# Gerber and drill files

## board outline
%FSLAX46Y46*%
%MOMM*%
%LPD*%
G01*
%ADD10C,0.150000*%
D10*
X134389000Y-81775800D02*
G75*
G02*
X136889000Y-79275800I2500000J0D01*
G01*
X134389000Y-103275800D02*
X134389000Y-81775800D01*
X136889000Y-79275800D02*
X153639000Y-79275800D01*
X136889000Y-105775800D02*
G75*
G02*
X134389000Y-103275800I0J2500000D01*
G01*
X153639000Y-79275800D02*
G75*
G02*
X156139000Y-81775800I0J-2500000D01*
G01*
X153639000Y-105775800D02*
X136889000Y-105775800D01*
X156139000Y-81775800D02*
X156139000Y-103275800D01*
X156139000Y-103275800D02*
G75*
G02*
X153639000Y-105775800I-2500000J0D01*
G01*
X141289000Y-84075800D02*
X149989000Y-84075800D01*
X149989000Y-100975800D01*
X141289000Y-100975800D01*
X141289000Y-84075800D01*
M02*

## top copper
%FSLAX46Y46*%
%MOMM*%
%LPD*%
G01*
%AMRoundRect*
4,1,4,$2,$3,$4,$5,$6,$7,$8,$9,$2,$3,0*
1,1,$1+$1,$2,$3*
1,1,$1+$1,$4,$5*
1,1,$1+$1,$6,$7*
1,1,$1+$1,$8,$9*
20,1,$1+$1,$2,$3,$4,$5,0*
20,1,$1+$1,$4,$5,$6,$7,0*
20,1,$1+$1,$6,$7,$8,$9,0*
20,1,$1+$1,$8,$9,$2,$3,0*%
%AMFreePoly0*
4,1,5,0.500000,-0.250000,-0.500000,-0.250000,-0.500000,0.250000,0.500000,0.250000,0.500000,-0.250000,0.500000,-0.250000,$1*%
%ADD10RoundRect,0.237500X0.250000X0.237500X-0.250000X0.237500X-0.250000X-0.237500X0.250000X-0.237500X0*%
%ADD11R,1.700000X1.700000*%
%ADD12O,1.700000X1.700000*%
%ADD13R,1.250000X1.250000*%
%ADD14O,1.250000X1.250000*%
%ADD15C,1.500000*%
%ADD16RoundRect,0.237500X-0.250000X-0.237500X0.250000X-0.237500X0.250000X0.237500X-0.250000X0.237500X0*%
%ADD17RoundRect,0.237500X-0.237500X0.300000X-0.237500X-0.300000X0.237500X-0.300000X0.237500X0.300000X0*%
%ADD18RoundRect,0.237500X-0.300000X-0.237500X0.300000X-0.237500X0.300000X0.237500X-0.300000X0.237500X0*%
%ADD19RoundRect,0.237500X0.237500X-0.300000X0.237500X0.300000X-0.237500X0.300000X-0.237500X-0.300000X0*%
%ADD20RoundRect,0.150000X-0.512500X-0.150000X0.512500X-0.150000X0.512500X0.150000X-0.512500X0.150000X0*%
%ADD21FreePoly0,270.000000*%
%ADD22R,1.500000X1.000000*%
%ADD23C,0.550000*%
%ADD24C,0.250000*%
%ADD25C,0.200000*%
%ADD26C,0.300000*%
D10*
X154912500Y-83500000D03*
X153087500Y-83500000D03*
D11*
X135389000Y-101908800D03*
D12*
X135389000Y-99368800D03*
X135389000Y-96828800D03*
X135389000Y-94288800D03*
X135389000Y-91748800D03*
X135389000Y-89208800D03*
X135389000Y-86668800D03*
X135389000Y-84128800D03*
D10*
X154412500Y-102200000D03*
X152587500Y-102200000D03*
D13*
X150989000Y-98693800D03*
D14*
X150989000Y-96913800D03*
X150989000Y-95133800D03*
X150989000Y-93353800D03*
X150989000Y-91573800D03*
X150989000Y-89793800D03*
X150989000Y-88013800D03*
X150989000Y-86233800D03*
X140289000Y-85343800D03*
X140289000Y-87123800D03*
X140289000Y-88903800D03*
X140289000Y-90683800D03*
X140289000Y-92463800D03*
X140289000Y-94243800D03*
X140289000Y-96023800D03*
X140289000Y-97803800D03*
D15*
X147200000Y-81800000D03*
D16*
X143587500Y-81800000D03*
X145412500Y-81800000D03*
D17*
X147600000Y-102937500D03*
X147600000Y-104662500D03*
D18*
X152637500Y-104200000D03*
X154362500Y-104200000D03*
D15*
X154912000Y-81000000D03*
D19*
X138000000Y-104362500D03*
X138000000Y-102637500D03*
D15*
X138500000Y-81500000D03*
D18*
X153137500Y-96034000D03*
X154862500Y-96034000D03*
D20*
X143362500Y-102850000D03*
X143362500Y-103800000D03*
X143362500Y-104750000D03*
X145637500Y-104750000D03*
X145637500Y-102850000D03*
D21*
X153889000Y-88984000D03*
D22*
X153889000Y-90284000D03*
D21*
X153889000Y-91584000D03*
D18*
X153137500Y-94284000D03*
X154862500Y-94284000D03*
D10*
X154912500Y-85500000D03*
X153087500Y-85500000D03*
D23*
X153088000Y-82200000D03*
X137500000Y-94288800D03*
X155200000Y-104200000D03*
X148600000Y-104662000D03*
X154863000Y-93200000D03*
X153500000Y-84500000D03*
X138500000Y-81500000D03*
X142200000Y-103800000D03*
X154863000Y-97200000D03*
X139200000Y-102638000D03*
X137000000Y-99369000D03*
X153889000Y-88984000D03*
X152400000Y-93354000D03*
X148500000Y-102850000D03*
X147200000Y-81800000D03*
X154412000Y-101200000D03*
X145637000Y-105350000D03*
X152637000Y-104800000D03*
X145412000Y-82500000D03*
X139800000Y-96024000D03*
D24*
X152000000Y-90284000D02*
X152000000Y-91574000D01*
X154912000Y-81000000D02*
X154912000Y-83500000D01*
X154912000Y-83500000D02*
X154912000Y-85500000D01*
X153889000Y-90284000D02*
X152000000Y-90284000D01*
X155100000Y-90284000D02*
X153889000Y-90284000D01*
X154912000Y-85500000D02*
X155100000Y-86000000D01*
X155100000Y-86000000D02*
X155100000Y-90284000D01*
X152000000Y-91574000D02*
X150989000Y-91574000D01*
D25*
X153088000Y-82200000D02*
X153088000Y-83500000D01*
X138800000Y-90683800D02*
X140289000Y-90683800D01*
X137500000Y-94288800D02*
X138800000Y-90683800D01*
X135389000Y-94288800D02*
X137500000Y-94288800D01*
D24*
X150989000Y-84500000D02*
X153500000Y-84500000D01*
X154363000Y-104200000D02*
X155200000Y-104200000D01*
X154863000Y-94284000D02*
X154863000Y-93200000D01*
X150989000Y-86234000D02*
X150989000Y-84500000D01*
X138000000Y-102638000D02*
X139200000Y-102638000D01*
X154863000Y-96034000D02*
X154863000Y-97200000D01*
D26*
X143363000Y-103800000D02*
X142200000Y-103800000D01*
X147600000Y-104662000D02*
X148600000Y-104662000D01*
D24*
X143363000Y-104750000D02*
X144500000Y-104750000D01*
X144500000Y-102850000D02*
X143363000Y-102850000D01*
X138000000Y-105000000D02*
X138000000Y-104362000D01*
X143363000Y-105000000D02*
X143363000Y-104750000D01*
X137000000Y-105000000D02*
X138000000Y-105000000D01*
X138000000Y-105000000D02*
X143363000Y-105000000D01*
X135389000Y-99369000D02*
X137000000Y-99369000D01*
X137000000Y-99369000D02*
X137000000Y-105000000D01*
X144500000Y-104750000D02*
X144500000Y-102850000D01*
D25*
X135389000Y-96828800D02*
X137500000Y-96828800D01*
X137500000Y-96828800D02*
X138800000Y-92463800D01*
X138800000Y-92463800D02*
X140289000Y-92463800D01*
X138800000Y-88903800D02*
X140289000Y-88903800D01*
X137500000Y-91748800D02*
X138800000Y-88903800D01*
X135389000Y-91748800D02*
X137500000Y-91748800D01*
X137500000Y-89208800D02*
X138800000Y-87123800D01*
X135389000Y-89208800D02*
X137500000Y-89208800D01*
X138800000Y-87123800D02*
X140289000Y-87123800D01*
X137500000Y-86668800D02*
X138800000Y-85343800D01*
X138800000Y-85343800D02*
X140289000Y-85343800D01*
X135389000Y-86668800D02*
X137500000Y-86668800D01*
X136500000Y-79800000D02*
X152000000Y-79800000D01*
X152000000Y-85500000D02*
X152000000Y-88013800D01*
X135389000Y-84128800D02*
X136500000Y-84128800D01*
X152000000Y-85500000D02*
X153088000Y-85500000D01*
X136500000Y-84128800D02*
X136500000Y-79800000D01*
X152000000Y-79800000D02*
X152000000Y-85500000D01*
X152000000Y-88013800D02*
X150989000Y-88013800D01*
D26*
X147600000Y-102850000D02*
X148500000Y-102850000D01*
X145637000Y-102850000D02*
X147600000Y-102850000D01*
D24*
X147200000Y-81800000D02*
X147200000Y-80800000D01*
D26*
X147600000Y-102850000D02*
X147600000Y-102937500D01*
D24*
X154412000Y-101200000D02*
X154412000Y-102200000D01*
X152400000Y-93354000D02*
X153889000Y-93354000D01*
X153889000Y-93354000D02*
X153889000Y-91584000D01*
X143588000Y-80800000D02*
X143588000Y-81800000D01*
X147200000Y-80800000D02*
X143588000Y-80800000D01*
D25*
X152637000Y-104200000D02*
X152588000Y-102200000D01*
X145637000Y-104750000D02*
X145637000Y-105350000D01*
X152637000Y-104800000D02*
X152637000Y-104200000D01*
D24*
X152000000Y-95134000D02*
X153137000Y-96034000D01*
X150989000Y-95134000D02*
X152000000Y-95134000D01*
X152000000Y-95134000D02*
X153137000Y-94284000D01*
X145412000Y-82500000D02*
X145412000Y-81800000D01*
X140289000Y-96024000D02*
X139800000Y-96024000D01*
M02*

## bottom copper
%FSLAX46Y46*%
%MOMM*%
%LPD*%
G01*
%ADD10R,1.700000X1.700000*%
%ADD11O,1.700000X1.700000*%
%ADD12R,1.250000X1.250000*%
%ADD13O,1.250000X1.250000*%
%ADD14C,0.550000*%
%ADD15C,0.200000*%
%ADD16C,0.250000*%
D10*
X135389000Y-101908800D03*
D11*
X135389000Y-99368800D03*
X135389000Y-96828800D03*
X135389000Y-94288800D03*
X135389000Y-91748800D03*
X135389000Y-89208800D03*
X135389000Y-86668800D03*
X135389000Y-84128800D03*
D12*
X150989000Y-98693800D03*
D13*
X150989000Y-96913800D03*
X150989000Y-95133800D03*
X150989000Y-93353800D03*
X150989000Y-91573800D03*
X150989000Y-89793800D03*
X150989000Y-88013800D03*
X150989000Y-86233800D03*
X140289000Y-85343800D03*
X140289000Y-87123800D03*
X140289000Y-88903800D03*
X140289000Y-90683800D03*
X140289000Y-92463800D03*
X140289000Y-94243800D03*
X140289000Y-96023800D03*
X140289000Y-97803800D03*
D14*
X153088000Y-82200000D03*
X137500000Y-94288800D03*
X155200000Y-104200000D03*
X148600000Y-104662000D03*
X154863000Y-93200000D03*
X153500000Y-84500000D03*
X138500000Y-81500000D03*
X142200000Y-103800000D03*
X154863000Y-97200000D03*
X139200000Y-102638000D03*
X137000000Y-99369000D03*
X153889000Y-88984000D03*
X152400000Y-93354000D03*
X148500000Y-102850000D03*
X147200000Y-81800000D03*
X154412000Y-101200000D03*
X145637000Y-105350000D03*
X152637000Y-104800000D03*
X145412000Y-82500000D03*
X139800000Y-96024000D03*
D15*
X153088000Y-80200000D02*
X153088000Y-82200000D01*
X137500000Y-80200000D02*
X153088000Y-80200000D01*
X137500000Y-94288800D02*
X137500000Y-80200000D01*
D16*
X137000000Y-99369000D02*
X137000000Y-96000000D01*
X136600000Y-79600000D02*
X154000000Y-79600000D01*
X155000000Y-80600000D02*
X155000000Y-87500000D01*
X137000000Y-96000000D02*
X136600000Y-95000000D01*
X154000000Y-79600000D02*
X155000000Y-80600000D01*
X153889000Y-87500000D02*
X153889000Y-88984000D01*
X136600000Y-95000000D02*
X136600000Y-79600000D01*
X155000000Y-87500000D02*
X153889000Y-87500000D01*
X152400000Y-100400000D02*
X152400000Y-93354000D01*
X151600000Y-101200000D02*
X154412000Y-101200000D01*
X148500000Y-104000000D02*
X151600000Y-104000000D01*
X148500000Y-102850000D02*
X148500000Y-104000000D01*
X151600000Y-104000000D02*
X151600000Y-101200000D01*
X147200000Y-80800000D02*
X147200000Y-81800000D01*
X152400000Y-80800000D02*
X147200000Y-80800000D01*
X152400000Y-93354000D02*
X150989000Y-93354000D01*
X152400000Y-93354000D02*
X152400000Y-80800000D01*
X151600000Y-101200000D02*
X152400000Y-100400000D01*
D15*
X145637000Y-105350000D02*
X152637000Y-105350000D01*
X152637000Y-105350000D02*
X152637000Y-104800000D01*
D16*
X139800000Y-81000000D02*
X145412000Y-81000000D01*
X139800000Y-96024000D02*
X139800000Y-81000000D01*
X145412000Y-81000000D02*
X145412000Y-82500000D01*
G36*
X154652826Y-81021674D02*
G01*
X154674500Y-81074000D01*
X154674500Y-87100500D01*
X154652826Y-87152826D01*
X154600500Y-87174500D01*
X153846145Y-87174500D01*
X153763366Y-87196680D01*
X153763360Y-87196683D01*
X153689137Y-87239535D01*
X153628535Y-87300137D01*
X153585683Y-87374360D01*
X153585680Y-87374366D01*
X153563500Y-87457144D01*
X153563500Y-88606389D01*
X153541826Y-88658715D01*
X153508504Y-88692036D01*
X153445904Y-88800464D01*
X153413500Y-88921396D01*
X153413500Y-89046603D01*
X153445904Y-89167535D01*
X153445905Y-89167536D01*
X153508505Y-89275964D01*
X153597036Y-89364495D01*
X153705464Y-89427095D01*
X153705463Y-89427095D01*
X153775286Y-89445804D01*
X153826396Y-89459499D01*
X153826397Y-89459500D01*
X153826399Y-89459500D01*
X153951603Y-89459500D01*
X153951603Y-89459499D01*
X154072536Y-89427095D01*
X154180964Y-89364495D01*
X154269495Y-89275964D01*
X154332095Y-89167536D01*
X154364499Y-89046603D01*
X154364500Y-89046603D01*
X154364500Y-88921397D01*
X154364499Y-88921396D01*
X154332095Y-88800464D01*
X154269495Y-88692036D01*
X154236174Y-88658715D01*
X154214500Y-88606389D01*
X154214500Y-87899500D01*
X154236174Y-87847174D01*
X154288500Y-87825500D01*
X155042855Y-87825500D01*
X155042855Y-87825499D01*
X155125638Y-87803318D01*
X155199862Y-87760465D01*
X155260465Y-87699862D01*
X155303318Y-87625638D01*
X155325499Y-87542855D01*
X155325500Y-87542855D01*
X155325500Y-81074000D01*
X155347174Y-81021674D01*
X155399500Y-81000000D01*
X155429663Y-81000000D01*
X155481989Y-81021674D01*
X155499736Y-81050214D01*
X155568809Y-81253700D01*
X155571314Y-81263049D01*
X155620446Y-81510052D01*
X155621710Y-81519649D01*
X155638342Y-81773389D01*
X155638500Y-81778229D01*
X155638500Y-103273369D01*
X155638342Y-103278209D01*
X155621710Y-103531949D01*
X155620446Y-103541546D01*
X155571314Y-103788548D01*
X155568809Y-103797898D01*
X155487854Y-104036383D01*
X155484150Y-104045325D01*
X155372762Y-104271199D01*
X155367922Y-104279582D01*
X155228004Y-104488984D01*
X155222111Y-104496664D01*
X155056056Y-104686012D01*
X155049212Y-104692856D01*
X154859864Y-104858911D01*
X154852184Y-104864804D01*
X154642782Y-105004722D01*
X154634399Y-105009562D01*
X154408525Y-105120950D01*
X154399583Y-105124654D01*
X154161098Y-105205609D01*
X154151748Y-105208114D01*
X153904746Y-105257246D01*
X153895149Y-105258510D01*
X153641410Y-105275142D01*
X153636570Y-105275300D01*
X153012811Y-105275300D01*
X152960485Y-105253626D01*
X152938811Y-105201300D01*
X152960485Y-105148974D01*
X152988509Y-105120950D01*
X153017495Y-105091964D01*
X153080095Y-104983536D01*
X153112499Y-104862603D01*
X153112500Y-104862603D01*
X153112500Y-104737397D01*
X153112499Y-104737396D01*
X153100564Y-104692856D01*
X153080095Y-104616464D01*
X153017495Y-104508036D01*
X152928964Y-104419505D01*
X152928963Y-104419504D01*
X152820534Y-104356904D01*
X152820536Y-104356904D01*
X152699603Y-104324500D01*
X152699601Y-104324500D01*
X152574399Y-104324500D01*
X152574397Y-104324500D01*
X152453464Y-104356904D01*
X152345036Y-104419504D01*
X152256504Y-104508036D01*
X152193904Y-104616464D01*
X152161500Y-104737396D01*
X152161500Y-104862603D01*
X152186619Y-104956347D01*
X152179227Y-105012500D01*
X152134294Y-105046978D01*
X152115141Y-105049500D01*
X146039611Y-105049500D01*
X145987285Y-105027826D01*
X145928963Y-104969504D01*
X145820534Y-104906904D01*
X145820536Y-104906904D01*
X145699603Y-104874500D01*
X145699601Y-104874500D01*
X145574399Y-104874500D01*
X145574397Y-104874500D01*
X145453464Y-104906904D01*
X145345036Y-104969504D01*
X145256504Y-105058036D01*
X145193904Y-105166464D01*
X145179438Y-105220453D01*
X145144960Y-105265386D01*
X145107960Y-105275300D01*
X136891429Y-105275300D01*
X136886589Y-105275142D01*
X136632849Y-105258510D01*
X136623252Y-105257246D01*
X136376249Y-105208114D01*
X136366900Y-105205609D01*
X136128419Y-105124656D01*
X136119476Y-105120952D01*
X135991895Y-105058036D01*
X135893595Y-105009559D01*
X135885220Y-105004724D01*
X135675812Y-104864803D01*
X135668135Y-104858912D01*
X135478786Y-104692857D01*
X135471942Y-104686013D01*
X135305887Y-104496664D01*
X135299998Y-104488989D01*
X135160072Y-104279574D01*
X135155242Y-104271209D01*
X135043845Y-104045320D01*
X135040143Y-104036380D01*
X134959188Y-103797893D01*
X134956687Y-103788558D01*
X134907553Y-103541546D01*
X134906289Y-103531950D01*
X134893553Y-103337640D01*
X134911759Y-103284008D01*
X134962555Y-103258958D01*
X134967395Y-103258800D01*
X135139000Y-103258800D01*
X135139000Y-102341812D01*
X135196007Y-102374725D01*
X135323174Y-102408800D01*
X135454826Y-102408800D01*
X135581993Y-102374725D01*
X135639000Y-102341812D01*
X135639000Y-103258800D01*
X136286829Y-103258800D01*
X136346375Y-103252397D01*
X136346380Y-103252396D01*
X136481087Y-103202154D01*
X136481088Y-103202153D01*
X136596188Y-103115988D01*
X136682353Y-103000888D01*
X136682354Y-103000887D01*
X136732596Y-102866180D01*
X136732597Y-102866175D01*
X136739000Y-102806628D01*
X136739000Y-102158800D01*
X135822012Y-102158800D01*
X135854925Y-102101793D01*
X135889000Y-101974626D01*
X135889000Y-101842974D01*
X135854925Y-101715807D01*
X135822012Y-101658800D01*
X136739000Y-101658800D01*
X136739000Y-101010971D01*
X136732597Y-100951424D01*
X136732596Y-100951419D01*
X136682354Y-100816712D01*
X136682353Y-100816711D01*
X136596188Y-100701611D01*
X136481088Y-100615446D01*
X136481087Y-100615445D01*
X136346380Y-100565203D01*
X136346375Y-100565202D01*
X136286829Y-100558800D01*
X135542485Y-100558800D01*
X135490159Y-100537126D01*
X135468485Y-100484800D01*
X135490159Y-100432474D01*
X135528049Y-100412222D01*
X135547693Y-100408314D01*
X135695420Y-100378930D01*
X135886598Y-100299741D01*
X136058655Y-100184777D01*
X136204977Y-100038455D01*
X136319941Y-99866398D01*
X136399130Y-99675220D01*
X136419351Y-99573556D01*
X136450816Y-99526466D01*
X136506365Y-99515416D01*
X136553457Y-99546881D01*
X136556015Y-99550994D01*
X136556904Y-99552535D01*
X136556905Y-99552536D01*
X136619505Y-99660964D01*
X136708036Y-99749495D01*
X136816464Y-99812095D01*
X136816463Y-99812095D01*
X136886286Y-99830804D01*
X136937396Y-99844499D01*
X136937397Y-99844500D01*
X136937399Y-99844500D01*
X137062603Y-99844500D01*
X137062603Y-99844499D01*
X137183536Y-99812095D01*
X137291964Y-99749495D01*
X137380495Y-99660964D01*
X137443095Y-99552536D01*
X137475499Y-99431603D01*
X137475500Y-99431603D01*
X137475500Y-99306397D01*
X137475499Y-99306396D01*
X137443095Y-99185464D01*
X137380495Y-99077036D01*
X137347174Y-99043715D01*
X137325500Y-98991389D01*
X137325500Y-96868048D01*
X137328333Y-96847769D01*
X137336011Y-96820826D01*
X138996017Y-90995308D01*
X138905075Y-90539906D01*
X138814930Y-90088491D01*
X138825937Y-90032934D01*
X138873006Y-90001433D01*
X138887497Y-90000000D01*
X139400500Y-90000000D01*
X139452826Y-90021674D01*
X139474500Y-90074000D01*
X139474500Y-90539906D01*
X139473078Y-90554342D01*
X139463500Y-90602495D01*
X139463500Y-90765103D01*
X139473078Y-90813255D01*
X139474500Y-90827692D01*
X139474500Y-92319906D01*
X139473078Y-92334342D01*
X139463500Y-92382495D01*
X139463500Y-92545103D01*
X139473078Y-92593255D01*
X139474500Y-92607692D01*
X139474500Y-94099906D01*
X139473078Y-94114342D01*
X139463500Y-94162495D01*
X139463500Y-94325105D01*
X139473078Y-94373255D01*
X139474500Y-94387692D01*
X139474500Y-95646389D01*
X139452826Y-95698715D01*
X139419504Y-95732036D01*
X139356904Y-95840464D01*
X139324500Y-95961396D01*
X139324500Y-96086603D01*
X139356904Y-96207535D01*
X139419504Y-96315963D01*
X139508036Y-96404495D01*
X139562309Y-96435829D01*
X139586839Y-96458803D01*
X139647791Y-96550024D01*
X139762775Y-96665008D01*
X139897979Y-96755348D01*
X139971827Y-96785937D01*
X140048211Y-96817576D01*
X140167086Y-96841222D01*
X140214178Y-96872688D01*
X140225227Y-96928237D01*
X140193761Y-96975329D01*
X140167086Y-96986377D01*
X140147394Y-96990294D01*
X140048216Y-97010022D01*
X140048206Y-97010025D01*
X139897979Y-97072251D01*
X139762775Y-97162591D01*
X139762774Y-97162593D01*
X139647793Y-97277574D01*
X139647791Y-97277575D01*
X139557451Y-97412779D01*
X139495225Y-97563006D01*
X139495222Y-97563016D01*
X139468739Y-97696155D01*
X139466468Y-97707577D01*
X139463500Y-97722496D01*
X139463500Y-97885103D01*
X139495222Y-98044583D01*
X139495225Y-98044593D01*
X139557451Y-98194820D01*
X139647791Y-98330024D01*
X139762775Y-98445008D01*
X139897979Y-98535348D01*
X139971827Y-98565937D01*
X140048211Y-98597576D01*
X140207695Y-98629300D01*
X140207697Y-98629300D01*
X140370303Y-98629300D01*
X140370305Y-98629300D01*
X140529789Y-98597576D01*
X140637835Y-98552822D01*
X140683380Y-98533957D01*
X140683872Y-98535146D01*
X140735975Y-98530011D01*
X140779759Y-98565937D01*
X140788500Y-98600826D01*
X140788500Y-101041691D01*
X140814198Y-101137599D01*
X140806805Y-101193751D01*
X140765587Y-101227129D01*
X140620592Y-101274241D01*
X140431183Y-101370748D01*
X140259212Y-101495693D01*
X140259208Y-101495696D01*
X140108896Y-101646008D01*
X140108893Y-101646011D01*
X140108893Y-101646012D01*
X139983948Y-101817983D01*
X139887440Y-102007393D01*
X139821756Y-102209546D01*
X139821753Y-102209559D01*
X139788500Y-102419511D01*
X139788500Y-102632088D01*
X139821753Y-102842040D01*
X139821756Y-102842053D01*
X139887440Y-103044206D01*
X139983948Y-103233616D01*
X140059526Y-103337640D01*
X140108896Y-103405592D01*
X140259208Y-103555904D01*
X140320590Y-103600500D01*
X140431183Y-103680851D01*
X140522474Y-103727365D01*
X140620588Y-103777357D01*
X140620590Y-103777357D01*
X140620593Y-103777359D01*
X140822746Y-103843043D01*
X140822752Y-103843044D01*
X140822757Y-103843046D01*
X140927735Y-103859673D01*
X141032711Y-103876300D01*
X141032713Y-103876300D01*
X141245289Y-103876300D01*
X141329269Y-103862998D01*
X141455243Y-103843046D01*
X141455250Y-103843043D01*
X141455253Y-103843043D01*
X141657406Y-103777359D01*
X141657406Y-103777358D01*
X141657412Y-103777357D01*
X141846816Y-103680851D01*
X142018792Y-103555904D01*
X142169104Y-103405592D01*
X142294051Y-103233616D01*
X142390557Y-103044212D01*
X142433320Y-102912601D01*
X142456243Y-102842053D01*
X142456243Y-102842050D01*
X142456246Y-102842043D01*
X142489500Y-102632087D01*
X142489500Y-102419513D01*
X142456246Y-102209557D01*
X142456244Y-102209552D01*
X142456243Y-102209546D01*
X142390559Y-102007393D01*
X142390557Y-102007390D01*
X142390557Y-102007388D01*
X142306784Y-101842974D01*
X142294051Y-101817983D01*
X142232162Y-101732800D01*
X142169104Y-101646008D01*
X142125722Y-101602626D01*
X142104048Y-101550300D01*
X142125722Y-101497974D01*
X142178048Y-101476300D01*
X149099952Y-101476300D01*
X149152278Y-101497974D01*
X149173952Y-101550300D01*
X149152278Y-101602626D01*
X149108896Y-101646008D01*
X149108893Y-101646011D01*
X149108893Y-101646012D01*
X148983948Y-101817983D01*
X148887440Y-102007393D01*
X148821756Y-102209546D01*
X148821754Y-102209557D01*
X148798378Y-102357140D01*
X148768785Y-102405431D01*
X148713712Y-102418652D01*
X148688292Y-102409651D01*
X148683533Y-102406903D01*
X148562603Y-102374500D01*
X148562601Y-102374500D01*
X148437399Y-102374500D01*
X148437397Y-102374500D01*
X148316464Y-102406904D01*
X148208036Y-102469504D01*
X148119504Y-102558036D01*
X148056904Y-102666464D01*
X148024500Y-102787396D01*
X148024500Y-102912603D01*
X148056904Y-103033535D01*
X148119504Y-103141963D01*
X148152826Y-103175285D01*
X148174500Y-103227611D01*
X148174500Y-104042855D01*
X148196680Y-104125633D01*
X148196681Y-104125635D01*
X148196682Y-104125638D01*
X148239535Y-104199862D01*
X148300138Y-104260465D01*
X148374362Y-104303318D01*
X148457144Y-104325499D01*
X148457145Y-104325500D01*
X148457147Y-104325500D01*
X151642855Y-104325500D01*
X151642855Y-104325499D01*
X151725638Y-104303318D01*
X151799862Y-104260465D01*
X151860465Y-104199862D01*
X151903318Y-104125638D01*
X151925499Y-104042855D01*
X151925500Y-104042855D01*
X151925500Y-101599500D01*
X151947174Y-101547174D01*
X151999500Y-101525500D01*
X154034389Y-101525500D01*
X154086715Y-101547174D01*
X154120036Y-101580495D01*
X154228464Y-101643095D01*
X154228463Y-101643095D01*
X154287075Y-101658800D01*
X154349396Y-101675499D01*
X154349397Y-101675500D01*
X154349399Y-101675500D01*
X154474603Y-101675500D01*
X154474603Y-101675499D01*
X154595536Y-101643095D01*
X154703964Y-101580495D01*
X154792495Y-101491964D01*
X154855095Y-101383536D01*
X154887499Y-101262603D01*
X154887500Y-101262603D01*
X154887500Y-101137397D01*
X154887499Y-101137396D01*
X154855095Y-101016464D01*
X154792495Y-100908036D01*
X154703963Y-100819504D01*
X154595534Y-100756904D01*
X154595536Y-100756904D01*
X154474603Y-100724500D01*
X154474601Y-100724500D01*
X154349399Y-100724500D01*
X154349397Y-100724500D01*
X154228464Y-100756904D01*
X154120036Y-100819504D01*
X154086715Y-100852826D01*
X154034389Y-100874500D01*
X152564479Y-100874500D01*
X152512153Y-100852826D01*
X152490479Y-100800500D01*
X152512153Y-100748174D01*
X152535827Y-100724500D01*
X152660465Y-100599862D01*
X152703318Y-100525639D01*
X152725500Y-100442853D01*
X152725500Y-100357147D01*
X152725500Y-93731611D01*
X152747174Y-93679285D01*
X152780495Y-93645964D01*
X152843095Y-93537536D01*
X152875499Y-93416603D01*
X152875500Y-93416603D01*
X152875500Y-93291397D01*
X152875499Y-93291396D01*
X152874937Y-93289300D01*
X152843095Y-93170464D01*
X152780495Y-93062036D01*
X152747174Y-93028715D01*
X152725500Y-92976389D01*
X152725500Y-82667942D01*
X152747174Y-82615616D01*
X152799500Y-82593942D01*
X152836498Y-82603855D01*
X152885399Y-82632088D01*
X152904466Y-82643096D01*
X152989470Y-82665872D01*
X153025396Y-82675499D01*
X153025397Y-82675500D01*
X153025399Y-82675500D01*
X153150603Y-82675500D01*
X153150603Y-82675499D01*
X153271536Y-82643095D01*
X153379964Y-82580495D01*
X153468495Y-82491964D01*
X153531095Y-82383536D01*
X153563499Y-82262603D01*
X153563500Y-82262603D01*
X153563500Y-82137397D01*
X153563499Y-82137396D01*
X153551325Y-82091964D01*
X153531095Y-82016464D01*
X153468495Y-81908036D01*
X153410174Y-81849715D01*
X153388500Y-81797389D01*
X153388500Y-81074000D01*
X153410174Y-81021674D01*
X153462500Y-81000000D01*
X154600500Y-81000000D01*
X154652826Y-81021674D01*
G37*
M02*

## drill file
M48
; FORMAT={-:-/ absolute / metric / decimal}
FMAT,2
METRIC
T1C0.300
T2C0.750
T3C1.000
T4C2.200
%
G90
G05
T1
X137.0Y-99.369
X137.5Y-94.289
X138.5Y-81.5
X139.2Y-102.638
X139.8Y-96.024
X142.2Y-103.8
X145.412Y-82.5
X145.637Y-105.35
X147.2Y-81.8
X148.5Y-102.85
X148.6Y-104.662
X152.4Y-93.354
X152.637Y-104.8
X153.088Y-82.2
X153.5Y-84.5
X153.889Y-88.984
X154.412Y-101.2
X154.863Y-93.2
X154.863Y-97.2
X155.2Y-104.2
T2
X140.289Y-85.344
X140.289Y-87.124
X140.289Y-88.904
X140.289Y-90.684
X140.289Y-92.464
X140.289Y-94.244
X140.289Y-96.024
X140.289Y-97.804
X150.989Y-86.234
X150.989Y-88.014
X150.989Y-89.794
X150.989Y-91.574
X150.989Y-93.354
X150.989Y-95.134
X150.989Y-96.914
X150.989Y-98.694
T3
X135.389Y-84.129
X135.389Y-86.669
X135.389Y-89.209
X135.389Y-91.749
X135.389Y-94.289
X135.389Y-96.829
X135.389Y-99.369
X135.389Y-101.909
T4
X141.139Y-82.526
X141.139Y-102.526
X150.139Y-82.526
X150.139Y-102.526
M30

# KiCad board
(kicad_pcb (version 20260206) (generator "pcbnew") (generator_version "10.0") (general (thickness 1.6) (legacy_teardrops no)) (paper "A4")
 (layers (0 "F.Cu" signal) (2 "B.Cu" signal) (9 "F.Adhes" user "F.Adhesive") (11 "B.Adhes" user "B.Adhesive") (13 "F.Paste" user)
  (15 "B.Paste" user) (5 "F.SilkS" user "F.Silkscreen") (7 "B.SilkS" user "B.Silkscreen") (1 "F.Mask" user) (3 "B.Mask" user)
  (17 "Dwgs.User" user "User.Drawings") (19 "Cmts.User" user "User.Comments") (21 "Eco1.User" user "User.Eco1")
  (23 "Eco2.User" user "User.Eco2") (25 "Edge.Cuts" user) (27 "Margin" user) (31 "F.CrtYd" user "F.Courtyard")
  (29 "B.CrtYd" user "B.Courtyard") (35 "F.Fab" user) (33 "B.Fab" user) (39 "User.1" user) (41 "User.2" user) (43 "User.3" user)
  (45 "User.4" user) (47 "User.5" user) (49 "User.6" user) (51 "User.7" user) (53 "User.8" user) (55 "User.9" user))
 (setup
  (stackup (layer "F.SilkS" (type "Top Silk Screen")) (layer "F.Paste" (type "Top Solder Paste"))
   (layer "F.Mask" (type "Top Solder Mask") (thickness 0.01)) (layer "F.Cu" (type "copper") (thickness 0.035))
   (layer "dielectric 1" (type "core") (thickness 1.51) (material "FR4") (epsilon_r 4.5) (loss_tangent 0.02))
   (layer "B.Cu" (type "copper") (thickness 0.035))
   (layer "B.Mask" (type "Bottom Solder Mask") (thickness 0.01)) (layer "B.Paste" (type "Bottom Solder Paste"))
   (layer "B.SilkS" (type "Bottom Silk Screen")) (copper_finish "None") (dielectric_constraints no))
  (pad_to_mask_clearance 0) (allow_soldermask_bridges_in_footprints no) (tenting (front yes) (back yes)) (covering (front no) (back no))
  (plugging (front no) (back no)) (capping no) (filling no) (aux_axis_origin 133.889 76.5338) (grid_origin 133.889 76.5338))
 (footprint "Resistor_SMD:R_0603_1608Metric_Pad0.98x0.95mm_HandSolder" (layer "F.Cu") (at 154 83.5 180)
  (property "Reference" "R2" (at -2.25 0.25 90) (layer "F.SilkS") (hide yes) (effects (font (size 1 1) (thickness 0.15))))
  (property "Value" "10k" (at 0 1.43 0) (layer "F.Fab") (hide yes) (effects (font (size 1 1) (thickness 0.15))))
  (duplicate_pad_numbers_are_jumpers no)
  (pad "1" smd roundrect (at -0.9125 0 180) (size 0.975 0.95) (layers "F.Cu" "F.Mask" "F.Paste") (roundrect_rratio 0.25) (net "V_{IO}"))
  (pad "2" smd roundrect (at 0.9125 0 180) (size 0.975 0.95) (layers "F.Cu" "F.Mask" "F.Paste") (roundrect_rratio 0.25) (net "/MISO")))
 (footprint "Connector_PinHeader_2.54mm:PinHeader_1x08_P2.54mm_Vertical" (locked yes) (layer "F.Cu") (at 135.389 101.9088 180)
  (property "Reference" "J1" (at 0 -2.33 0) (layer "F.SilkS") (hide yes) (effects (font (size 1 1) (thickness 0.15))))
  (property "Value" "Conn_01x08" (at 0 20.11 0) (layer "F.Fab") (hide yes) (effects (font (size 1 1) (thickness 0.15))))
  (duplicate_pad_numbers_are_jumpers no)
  (pad "1" thru_hole rect (at 0 0 180) (size 1.7 1.7) (drill 1) (layers "*.Cu" "*.Mask") (remove_unused_layers no) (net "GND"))
  (pad "2" thru_hole oval (at 0 2.54 180) (size 1.7 1.7) (drill 1) (layers "*.Cu" "*.Mask") (remove_unused_layers no) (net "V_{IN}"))
  (pad "3" thru_hole oval (at 0 5.08 180) (size 1.7 1.7) (drill 1) (layers "*.Cu" "*.Mask") (remove_unused_layers no) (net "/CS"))
  (pad "4" thru_hole oval (at 0 7.62 180) (size 1.7 1.7) (drill 1) (layers "*.Cu" "*.Mask") (remove_unused_layers no) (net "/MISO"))
  (pad "5" thru_hole oval (at 0 10.16 180) (size 1.7 1.7) (drill 1) (layers "*.Cu" "*.Mask") (remove_unused_layers no) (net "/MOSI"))
  (pad "6" thru_hole oval (at 0 12.7 180) (size 1.7 1.7) (drill 1) (layers "*.Cu" "*.Mask") (remove_unused_layers no) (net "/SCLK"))
  (pad "7" thru_hole oval (at 0 15.24 180) (size 1.7 1.7) (drill 1) (layers "*.Cu" "*.Mask") (remove_unused_layers no) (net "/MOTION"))
  (pad "8" thru_hole oval (at 0 17.78 180) (size 1.7 1.7) (drill 1) (layers "*.Cu" "*.Mask") (remove_unused_layers no) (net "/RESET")))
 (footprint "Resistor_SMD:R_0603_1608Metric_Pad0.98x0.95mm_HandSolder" (layer "F.Cu") (at 153.5 102.2 180)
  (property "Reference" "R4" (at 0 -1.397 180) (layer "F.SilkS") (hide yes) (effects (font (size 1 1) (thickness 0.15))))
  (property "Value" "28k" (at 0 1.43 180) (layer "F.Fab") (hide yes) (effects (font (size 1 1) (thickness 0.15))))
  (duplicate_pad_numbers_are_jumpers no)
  (pad "1" smd roundrect (at -0.9125 0 180) (size 0.975 0.95) (layers "F.Cu" "F.Mask" "F.Paste") (roundrect_rratio 0.25) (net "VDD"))
  (pad "2" smd roundrect (at 0.9125 0 180) (size 0.975 0.95) (layers "F.Cu" "F.Mask" "F.Paste") (roundrect_rratio 0.25) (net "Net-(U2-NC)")))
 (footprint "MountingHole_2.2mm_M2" (layer "F.Cu") (at 150.139 82.5258)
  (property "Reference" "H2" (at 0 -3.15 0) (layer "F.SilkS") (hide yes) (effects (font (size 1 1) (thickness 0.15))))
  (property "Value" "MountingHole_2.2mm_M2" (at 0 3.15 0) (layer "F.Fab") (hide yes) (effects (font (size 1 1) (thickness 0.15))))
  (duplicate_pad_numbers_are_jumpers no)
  (pad "" np_thru_hole circle (at 0 0) (size 2.2 2.2) (drill 2.2) (layers "*.Cu" "*.Mask")))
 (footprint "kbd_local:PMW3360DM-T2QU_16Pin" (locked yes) (layer "F.Cu") (at 145.639 92.5258 90)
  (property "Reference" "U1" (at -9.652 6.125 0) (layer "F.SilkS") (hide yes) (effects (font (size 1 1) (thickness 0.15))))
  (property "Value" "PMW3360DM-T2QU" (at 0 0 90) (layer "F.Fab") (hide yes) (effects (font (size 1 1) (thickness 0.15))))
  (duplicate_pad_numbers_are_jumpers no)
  (fp_rect (start 8.45 -4.35) (end -8.45 4.35) (stroke (width 0.15) (type solid)) (fill no) (layer "Edge.Cuts"))
  (pad "1" thru_hole rect (at -6.168 5.35 90) (size 1.25 1.25) (drill 0.75) (layers "*.Cu" "*.Mask") (remove_unused_layers no)
   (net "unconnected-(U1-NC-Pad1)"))
  (pad "2" thru_hole oval (at -4.388 5.35 90) (size 1.25 1.25) (drill 0.75) (layers "*.Cu" "*.Mask") (remove_unused_layers no)
   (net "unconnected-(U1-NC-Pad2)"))
  (pad "3" thru_hole oval (at -2.608 5.35 90) (size 1.25 1.25) (drill 0.75) (layers "*.Cu" "*.Mask") (remove_unused_layers no)
   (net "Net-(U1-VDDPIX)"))
  (pad "4" thru_hole oval (at -0.828 5.35 90) (size 1.25 1.25) (drill 0.75) (layers "*.Cu" "*.Mask") (remove_unused_layers no) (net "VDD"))
  (pad "5" thru_hole oval (at 0.952 5.35 90) (size 1.25 1.25) (drill 0.75) (layers "*.Cu" "*.Mask") (remove_unused_layers no) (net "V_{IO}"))
  (pad "6" thru_hole oval (at 2.732 5.35 90) (size 1.25 1.25) (drill 0.75) (layers "*.Cu" "*.Mask") (remove_unused_layers no)
   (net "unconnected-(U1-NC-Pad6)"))
  (pad "7" thru_hole oval (at 4.512 5.35 90) (size 1.25 1.25) (drill 0.75) (layers "*.Cu" "*.Mask") (remove_unused_layers no) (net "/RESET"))
  (pad "8" thru_hole oval (at 6.292 5.35 90) (size 1.25 1.25) (drill 0.75) (layers "*.Cu" "*.Mask") (remove_unused_layers no) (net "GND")
   (zone_connect 2))
  (pad "9" thru_hole oval (at 7.182 -5.35 90) (size 1.25 1.25) (drill 0.75) (layers "*.Cu" "*.Mask") (remove_unused_layers no)
   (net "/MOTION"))
  (pad "10" thru_hole oval (at 5.402 -5.35 90) (size 1.25 1.25) (drill 0.75) (layers "*.Cu" "*.Mask") (remove_unused_layers no)
   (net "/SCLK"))
  (pad "11" thru_hole oval (at 3.622 -5.35 90) (size 1.25 1.25) (drill 0.75) (layers "*.Cu" "*.Mask") (remove_unused_layers no)
   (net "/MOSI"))
  (pad "12" thru_hole oval (at 1.842 -5.35 90) (size 1.25 1.25) (drill 0.75) (layers "*.Cu" "*.Mask") (remove_unused_layers no)
   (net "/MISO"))
  (pad "13" thru_hole oval (at 0.062 -5.35 90) (size 1.25 1.25) (drill 0.75) (layers "*.Cu" "*.Mask") (remove_unused_layers no) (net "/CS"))
  (pad "14" thru_hole oval (at -1.718 -5.35 90) (size 1.25 1.25) (drill 0.75) (layers "*.Cu" "*.Mask") (remove_unused_layers no)
   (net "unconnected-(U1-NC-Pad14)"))
  (pad "15" thru_hole oval (at -3.498 -5.35 90) (size 1.25 1.25) (drill 0.75) (layers "*.Cu" "*.Mask") (remove_unused_layers no)
   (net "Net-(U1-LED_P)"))
  (pad "16" thru_hole oval (at -5.278 -5.35 90) (size 1.25 1.25) (drill 0.75) (layers "*.Cu" "*.Mask") (remove_unused_layers no)
   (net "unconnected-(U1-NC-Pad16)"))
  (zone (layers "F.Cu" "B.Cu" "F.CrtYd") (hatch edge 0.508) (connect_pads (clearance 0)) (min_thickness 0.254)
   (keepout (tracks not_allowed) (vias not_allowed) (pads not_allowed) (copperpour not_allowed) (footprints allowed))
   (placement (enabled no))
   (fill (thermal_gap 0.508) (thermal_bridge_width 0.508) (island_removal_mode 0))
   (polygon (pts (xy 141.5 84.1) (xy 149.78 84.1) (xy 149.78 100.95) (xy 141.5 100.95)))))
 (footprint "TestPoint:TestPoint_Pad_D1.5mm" (layer "F.Cu") (at 147.2 81.8)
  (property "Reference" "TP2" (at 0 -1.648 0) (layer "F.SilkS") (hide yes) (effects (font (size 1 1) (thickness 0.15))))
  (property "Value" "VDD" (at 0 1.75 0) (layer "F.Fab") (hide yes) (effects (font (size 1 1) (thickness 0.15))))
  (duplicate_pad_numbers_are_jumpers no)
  (pad "1" smd circle (at 0 0) (size 1.5 1.5) (layers "F.Cu" "F.Mask") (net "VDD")))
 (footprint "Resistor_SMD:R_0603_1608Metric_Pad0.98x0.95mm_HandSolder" (layer "F.Cu") (at 144.5 81.8)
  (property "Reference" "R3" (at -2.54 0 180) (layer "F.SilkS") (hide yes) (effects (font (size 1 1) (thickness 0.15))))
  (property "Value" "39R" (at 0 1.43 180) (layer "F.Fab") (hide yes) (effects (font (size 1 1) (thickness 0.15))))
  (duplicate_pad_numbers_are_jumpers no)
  (pad "1" smd roundrect (at -0.9125 0) (size 0.975 0.95) (layers "F.Cu" "F.Mask" "F.Paste") (roundrect_rratio 0.25) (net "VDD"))
  (pad "2" smd roundrect (at 0.9125 0) (size 0.975 0.95) (layers "F.Cu" "F.Mask" "F.Paste") (roundrect_rratio 0.25) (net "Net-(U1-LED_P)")))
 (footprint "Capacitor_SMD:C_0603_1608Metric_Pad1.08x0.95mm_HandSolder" (layer "F.Cu") (at 147.6 103.8 -90)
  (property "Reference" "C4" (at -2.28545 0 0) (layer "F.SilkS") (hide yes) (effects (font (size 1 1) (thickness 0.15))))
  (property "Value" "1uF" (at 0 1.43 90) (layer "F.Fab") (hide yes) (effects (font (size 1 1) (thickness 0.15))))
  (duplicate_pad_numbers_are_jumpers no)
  (pad "1" smd roundrect (at -0.8625 0 270) (size 1.075 0.95) (layers "F.Cu" "F.Mask" "F.Paste") (roundrect_rratio 0.25) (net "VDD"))
  (pad "2" smd roundrect (at 0.8625 0 270) (size 1.075 0.95) (layers "F.Cu" "F.Mask" "F.Paste") (roundrect_rratio 0.25) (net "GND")))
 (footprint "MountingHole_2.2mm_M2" (layer "F.Cu") (at 150.139 102.5258)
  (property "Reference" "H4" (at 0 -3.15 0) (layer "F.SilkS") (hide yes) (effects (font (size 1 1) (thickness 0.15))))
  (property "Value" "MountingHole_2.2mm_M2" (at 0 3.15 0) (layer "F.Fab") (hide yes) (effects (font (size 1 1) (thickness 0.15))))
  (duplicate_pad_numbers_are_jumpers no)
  (pad "" np_thru_hole circle (at 0 0) (size 2.2 2.2) (drill 2.2) (layers "*.Cu" "*.Mask")))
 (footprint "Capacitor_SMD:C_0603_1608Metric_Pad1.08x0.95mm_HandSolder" (layer "F.Cu") (at 153.5 104.2)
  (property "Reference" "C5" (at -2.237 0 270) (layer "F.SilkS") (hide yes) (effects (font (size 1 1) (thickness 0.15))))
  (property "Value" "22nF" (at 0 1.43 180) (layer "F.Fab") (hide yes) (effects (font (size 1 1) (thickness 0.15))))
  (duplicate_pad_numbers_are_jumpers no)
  (pad "1" smd roundrect (at -0.8625 0) (size 1.075 0.95) (layers "F.Cu" "F.Mask" "F.Paste") (roundrect_rratio 0.25) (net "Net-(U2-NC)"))
  (pad "2" smd roundrect (at 0.8625 0) (size 1.075 0.95) (layers "F.Cu" "F.Mask" "F.Paste") (roundrect_rratio 0.25) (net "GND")))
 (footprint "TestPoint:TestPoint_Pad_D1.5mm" (layer "F.Cu") (at 154.912 81)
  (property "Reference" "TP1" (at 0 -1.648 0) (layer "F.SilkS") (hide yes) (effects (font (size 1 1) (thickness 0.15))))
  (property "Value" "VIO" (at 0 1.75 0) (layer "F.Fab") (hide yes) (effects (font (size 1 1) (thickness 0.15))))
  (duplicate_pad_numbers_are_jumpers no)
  (pad "1" smd circle (at 0 0) (size 1.5 1.5) (layers "F.Cu" "F.Mask") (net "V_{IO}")))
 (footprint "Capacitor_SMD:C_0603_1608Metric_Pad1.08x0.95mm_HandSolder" (layer "F.Cu") (at 138 103.5 90)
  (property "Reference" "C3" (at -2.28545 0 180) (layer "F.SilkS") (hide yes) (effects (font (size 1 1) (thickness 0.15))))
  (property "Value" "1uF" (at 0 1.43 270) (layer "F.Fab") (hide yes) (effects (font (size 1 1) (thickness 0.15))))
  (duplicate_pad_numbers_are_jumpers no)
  (pad "1" smd roundrect (at -0.8625 0 90) (size 1.075 0.95) (layers "F.Cu" "F.Mask" "F.Paste") (roundrect_rratio 0.25) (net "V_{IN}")
   (clearance 0.135))
  (pad "2" smd roundrect (at 0.8625 0 90) (size 1.075 0.95) (layers "F.Cu" "F.Mask" "F.Paste") (roundrect_rratio 0.25) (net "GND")
   (clearance 0.135)))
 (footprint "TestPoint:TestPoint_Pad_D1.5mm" (layer "F.Cu") (at 138.5 81.5)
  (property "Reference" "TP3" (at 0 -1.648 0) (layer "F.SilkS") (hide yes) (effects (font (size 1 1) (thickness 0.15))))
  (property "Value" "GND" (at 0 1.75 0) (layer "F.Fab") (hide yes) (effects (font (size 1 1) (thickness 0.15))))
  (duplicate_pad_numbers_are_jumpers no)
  (pad "1" smd circle (at 0 0) (size 1.5 1.5) (layers "F.Cu" "F.Mask") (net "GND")))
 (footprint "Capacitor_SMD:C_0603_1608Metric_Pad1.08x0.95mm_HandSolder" (layer "F.Cu") (at 154 96.034)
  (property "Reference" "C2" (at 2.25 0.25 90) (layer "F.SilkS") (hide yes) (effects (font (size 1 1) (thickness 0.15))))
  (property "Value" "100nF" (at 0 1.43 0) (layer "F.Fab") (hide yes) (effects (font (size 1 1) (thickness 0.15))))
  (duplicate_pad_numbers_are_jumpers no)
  (pad "1" smd roundrect (at -0.8625 0) (size 1.075 0.95) (layers "F.Cu" "F.Mask" "F.Paste") (roundrect_rratio 0.25) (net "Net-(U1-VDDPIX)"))
  (pad "2" smd roundrect (at 0.8625 0) (size 1.075 0.95) (layers "F.Cu" "F.Mask" "F.Paste") (roundrect_rratio 0.25) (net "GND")))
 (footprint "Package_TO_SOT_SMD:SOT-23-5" (layer "F.Cu") (at 144.5 103.8)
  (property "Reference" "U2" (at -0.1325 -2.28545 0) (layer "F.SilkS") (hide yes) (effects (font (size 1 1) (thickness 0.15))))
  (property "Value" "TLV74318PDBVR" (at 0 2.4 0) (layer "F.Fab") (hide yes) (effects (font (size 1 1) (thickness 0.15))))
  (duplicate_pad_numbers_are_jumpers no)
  (pad "1" smd roundrect (at -1.1375 -0.95) (size 1.325 0.6) (layers "F.Cu" "F.Mask" "F.Paste") (roundrect_rratio 0.25) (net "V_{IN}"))
  (pad "2" smd roundrect (at -1.1375 0) (size 1.325 0.6) (layers "F.Cu" "F.Mask" "F.Paste") (roundrect_rratio 0.25) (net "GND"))
  (pad "3" smd roundrect (at -1.1375 0.95) (size 1.325 0.6) (layers "F.Cu" "F.Mask" "F.Paste") (roundrect_rratio 0.25) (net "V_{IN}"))
  (pad "4" smd roundrect (at 1.1375 0.95) (size 1.325 0.6) (layers "F.Cu" "F.Mask" "F.Paste") (roundrect_rratio 0.25) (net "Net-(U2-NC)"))
  (pad "5" smd roundrect (at 1.1375 -0.95) (size 1.325 0.6) (layers "F.Cu" "F.Mask" "F.Paste") (roundrect_rratio 0.25) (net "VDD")))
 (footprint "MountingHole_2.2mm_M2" (layer "F.Cu") (at 141.139 82.5258)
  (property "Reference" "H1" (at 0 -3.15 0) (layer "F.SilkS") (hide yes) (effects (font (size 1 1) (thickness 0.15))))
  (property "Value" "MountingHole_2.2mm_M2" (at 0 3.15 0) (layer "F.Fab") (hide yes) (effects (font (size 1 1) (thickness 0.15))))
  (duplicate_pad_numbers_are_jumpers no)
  (pad "" np_thru_hole circle (at 0 0) (size 2.2 2.2) (drill 2.2) (layers "*.Cu" "*.Mask")))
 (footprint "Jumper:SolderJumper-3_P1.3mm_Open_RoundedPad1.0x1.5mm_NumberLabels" (layer "F.Cu") (at 153.889 90.284 -90)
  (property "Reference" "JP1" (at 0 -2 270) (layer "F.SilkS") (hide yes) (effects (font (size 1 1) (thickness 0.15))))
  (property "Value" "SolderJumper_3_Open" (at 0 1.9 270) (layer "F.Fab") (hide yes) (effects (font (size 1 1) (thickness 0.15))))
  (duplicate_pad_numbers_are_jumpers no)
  (pad "1" smd custom (at -1.3 0 270) (size 1 0.5) (layers "F.Cu" "F.Mask") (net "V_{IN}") (zone_connect 2) (thermal_bridge_angle 45)
   (options (clearance outline) (anchor rect)) (primitives))
  (pad "2" smd rect (at 0 0 270) (size 1 1.5) (layers "F.Cu" "F.Mask") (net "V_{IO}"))
  (pad "3" smd custom (at 1.3 0 270) (size 1 0.5) (layers "F.Cu" "F.Mask") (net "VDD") (zone_connect 2) (thermal_bridge_angle 45)
   (options (clearance outline) (anchor rect)) (primitives)))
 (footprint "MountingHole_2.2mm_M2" (layer "F.Cu") (at 141.139 102.5258)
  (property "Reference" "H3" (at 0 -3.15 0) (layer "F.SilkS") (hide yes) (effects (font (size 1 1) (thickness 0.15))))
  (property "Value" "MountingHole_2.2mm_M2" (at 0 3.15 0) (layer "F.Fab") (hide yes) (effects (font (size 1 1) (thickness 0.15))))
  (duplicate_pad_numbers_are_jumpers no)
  (pad "" np_thru_hole circle (at 0 0) (size 2.2 2.2) (drill 2.2) (layers "*.Cu" "*.Mask")))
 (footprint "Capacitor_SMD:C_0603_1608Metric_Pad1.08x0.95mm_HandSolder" (layer "F.Cu") (at 154 94.284)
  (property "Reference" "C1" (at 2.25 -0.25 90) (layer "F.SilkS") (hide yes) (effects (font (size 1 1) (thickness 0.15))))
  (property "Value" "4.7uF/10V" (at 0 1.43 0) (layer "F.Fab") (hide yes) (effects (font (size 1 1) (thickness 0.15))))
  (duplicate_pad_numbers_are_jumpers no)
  (pad "1" smd roundrect (at -0.8625 0) (size 1.075 0.95) (layers "F.Cu" "F.Mask" "F.Paste") (roundrect_rratio 0.25) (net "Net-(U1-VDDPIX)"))
  (pad "2" smd roundrect (at 0.8625 0) (size 1.075 0.95) (layers "F.Cu" "F.Mask" "F.Paste") (roundrect_rratio 0.25) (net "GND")))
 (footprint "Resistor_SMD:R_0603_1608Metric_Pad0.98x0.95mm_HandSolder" (layer "F.Cu") (at 154 85.5 180)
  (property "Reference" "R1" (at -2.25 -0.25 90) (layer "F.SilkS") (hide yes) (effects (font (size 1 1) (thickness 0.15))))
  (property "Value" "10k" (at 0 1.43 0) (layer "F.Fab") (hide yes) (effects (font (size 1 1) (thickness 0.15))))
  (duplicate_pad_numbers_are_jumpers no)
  (pad "1" smd roundrect (at -0.9125 0 180) (size 0.975 0.95) (layers "F.Cu" "F.Mask" "F.Paste") (roundrect_rratio 0.25) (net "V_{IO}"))
  (pad "2" smd roundrect (at 0.9125 0 180) (size 0.975 0.95) (layers "F.Cu" "F.Mask" "F.Paste") (roundrect_rratio 0.25) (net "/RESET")))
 (gr_arc (start 134.389 81.7758) (mid 135.121233 80.008033) (end 136.889 79.2758) (stroke (width 0.15) (type default)) (layer "Edge.Cuts"))
 (gr_line (start 134.389 103.2758) (end 134.389 81.7758) (stroke (width 0.15) (type default)) (layer "Edge.Cuts"))
 (gr_line (start 136.889 79.2758) (end 153.639 79.2758) (stroke (width 0.15) (type default)) (layer "Edge.Cuts"))
 (gr_arc (start 136.889 105.7758) (mid 135.121233 105.043566) (end 134.389 103.2758) (stroke (width 0.15) (type default))
  (layer "Edge.Cuts"))
 (gr_arc (start 153.639 79.2758) (mid 155.406766 80.008033) (end 156.139 81.7758) (stroke (width 0.15) (type default)) (layer "Edge.Cuts"))
 (gr_line (start 153.639 105.7758) (end 136.889 105.7758) (stroke (width 0.15) (type default)) (layer "Edge.Cuts"))
 (gr_line (start 156.139 81.7758) (end 156.139 103.2758) (stroke (width 0.15) (type default)) (layer "Edge.Cuts"))
 (gr_arc (start 156.139 103.2758) (mid 155.406766 105.043566) (end 153.639 105.7758) (stroke (width 0.15) (type default))
  (layer "Edge.Cuts"))
 (segment (start 152 90.284) (end 152 91.574) (width 0.25) (layer "F.Cu") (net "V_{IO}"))
 (segment (start 154.912 81) (end 154.912 83.5) (width 0.25) (layer "F.Cu") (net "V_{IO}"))
 (segment (start 154.912 83.5) (end 154.912 85.5) (width 0.25) (layer "F.Cu") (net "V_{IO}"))
 (segment (start 153.889 90.284) (end 152 90.284) (width 0.25) (layer "F.Cu") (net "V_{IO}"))
 (segment (start 155.1 90.284) (end 153.889 90.284) (width 0.25) (layer "F.Cu") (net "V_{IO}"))
 (segment (start 154.912 85.5) (end 155.1 86) (width 0.25) (layer "F.Cu") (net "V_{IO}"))
 (segment (start 155.1 86) (end 155.1 90.284) (width 0.25) (layer "F.Cu") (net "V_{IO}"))
 (segment (start 152 91.574) (end 150.989 91.574) (width 0.25) (layer "F.Cu") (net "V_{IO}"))
 (segment (start 153.088 82.2) (end 153.088 83.5) (width 0.2) (layer "F.Cu") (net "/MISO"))
 (segment (start 138.8 90.6838) (end 140.289 90.6838) (width 0.2) (layer "F.Cu") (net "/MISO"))
 (segment (start 137.5 94.2888) (end 138.8 90.6838) (width 0.2) (layer "F.Cu") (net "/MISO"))
 (segment (start 135.389 94.2888) (end 137.5 94.2888) (width 0.2) (layer "F.Cu") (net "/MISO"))
 (via (at 153.088 82.2) (size 0.55) (drill 0.3) (layers "F.Cu" "B.Cu") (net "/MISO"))
 (via (at 137.5 94.2888) (size 0.55) (drill 0.3) (layers "F.Cu" "B.Cu") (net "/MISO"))
 (segment (start 153.088 80.2) (end 153.088 82.2) (width 0.2) (layer "B.Cu") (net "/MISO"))
 (segment (start 137.5 80.2) (end 153.088 80.2) (width 0.2) (layer "B.Cu") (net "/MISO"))
 (segment (start 137.5 94.2888) (end 137.5 80.2) (width 0.2) (layer "B.Cu") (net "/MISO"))
 (segment (start 150.989 84.5) (end 153.5 84.5) (width 0.25) (layer "F.Cu") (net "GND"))
 (segment (start 154.363 104.2) (end 155.2 104.2) (width 0.25) (layer "F.Cu") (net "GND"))
 (segment (start 154.863 94.284) (end 154.863 93.2) (width 0.25) (layer "F.Cu") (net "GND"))
 (segment (start 150.989 86.234) (end 150.989 84.5) (width 0.25) (layer "F.Cu") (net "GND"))
 (segment (start 138 102.638) (end 139.2 102.638) (width 0.25) (layer "F.Cu") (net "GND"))
 (segment (start 154.863 96.034) (end 154.863 97.2) (width 0.25) (layer "F.Cu") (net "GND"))
 (segment (start 143.363 103.8) (end 142.2 103.8) (width 0.3) (layer "F.Cu") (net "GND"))
 (segment (start 147.6 104.662) (end 148.6 104.662) (width 0.3) (layer "F.Cu") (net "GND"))
 (via (at 155.2 104.2) (size 0.55) (drill 0.3) (layers "F.Cu" "B.Cu") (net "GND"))
 (via (at 148.6 104.662) (size 0.55) (drill 0.3) (layers "F.Cu" "B.Cu") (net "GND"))
 (via (at 154.863 93.2) (size 0.55) (drill 0.3) (layers "F.Cu" "B.Cu") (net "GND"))
 (via (at 153.5 84.5) (size 0.55) (drill 0.3) (layers "F.Cu" "B.Cu") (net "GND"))
 (via (at 138.5 81.5) (size 0.55) (drill 0.3) (layers "F.Cu" "B.Cu") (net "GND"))
 (via (at 142.2 103.8) (size 0.55) (drill 0.3) (layers "F.Cu" "B.Cu") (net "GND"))
 (via (at 154.863 97.2) (size 0.55) (drill 0.3) (layers "F.Cu" "B.Cu") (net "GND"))
 (via (at 139.2 102.638) (size 0.55) (drill 0.3) (layers "F.Cu" "B.Cu") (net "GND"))
 (segment (start 143.363 104.75) (end 144.5 104.75) (width 0.25) (layer "F.Cu") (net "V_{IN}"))
 (segment (start 144.5 102.85) (end 143.363 102.85) (width 0.25) (layer "F.Cu") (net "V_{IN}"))
 (segment (start 138 105) (end 138 104.362) (width 0.25) (layer "F.Cu") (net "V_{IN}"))
 (segment (start 143.363 105) (end 143.363 104.75) (width 0.25) (layer "F.Cu") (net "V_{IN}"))
 (segment (start 137 105) (end 138 105) (width 0.25) (layer "F.Cu") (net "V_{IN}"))
 (segment (start 138 105) (end 143.363 105) (width 0.25) (layer "F.Cu") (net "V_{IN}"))
 (segment (start 135.389 99.369) (end 137 99.369) (width 0.25) (layer "F.Cu") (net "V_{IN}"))
 (segment (start 137 99.369) (end 137 105) (width 0.25) (layer "F.Cu") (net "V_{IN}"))
 (segment (start 144.5 104.75) (end 144.5 102.85) (width 0.25) (layer "F.Cu") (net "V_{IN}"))
 (via (at 137 99.369) (size 0.55) (drill 0.3) (layers "F.Cu" "B.Cu") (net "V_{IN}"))
 (via (at 153.889 88.984) (size 0.55) (drill 0.3) (layers "F.Cu" "B.Cu") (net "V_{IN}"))
 (segment (start 137 99.369) (end 137 96) (width 0.25) (layer "B.Cu") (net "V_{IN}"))
 (segment (start 136.6 79.6) (end 154 79.6) (width 0.25) (layer "B.Cu") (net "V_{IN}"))
 (segment (start 155 80.6) (end 155 87.5) (width 0.25) (layer "B.Cu") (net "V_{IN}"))
 (segment (start 137 96) (end 136.6 95) (width 0.25) (layer "B.Cu") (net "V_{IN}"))
 (segment (start 154 79.6) (end 155 80.6) (width 0.25) (layer "B.Cu") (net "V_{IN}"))
 (segment (start 153.889 87.5) (end 153.889 88.984) (width 0.25) (layer "B.Cu") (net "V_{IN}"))
 (segment (start 136.6 95) (end 136.6 79.6) (width 0.25) (layer "B.Cu") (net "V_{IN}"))
 (segment (start 155 87.5) (end 153.889 87.5) (width 0.25) (layer "B.Cu") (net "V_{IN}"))
 (segment (start 135.389 96.8288) (end 137.5 96.8288) (width 0.2) (layer "F.Cu") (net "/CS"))
 (segment (start 137.5 96.8288) (end 138.8 92.4638) (width 0.2) (layer "F.Cu") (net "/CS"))
 (segment (start 138.8 92.4638) (end 140.289 92.4638) (width 0.2) (layer "F.Cu") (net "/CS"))
 (segment (start 138.8 88.9038) (end 140.289 88.9038) (width 0.2) (layer "F.Cu") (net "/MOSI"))
 (segment (start 137.5 91.7488) (end 138.8 88.9038) (width 0.2) (layer "F.Cu") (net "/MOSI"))
 (segment (start 135.389 91.7488) (end 137.5 91.7488) (width 0.2) (layer "F.Cu") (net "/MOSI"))
 (segment (start 137.5 89.2088) (end 138.8 87.1238) (width 0.2) (layer "F.Cu") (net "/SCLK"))
 (segment (start 135.389 89.2088) (end 137.5 89.2088) (width 0.2) (layer "F.Cu") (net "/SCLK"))
 (segment (start 138.8 87.1238) (end 140.289 87.1238) (width 0.2) (layer "F.Cu") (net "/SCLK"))
 (segment (start 137.5 86.6688) (end 138.8 85.3438) (width 0.2) (layer "F.Cu") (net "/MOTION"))
 (segment (start 138.8 85.3438) (end 140.289 85.3438) (width 0.2) (layer "F.Cu") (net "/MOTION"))
 (segment (start 135.389 86.6688) (end 137.5 86.6688) (width 0.2) (layer "F.Cu") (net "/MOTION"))
 (segment (start 136.5 79.8) (end 152 79.8) (width 0.2) (layer "F.Cu") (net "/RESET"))
 (segment (start 152 85.5) (end 152 88.0138) (width 0.2) (layer "F.Cu") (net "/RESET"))
 (segment (start 135.389 84.1288) (end 136.5 84.1288) (width 0.2) (layer "F.Cu") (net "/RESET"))
 (segment (start 152 85.5) (end 153.088 85.5) (width 0.2) (layer "F.Cu") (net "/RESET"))
 (segment (start 136.5 84.1288) (end 136.5 79.8) (width 0.2) (layer "F.Cu") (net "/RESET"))
 (segment (start 152 79.8) (end 152 85.5) (width 0.2) (layer "F.Cu") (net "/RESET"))
 (segment (start 152 88.0138) (end 150.989 88.0138) (width 0.2) (layer "F.Cu") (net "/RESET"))
 (segment (start 147.6 102.85) (end 148.5 102.85) (width 0.3) (layer "F.Cu") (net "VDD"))
 (segment (start 145.637 102.85) (end 147.6 102.85) (width 0.3) (layer "F.Cu") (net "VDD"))
 (segment (start 147.2 81.8) (end 147.2 80.8) (width 0.25) (layer "F.Cu") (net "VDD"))
 (segment (start 147.6 102.85) (end 147.6 102.9375) (width 0.3) (layer "F.Cu") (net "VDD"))
 (segment (start 154.412 101.2) (end 154.412 102.2) (width 0.25) (layer "F.Cu") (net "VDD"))
 (segment (start 152.4 93.354) (end 153.889 93.354) (width 0.25) (layer "F.Cu") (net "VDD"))
 (segment (start 153.889 93.354) (end 153.889 91.584) (width 0.25) (layer "F.Cu") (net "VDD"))
 (segment (start 143.588 80.8) (end 143.588 81.8) (width 0.25) (layer "F.Cu") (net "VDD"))
 (segment (start 147.2 80.8) (end 143.588 80.8) (width 0.25) (layer "F.Cu") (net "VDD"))
 (via (at 152.4 93.354) (size 0.55) (drill 0.3) (layers "F.Cu" "B.Cu") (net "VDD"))
 (via (at 148.5 102.85) (size 0.55) (drill 0.3) (layers "F.Cu" "B.Cu") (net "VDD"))
 (via (at 147.2 81.8) (size 0.55) (drill 0.3) (layers "F.Cu" "B.Cu") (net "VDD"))
 (via (at 154.412 101.2) (size 0.55) (drill 0.3) (layers "F.Cu" "B.Cu") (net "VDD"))
 (segment (start 152.4 100.4) (end 152.4 93.354) (width 0.25) (layer "B.Cu") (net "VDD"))
 (segment (start 151.6 101.2) (end 154.412 101.2) (width 0.25) (layer "B.Cu") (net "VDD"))
 (segment (start 148.5 104) (end 151.6 104) (width 0.25) (layer "B.Cu") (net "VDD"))
 (segment (start 148.5 102.85) (end 148.5 104) (width 0.25) (layer "B.Cu") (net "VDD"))
 (segment (start 151.6 104) (end 151.6 101.2) (width 0.25) (layer "B.Cu") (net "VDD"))
 (segment (start 147.2 80.8) (end 147.2 81.8) (width 0.25) (layer "B.Cu") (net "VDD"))
 (segment (start 152.4 80.8) (end 147.2 80.8) (width 0.25) (layer "B.Cu") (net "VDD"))
 (segment (start 152.4 93.354) (end 150.989 93.354) (width 0.25) (layer "B.Cu") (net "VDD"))
 (segment (start 152.4 93.354) (end 152.4 80.8) (width 0.25) (layer "B.Cu") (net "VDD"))
 (segment (start 151.6 101.2) (end 152.4 100.4) (width 0.25) (layer "B.Cu") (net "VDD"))
 (segment (start 152.637 104.2) (end 152.588 102.2) (width 0.2) (layer "F.Cu") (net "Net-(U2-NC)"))
 (segment (start 145.637 104.75) (end 145.637 105.35) (width 0.2) (layer "F.Cu") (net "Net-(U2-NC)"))
 (segment (start 152.637 104.8) (end 152.637 104.2) (width 0.2) (layer "F.Cu") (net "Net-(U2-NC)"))
 (via (at 145.637 105.35) (size 0.55) (drill 0.3) (layers "F.Cu" "B.Cu") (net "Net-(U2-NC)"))
 (via (at 152.637 104.8) (size 0.55) (drill 0.3) (layers "F.Cu" "B.Cu") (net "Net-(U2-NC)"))
 (segment (start 145.637 105.35) (end 152.637 105.35) (width 0.2) (layer "B.Cu") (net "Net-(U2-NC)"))
 (segment (start 152.637 105.35) (end 152.637 104.8) (width 0.2) (layer "B.Cu") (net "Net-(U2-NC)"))
 (segment (start 152 95.134) (end 153.137 96.034) (width 0.25) (layer "F.Cu") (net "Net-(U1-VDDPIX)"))
 (segment (start 150.989 95.134) (end 152 95.134) (width 0.25) (layer "F.Cu") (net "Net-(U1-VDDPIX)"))
 (segment (start 152 95.134) (end 153.137 94.284) (width 0.25) (layer "F.Cu") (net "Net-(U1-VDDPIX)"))
 (segment (start 145.412 82.5) (end 145.412 81.8) (width 0.25) (layer "F.Cu") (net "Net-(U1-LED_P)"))
 (segment (start 140.289 96.024) (end 139.8 96.024) (width 0.25) (layer "F.Cu") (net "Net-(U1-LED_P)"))
 (via (at 145.412 82.5) (size 0.55) (drill 0.3) (layers "F.Cu" "B.Cu") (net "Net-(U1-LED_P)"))
 (via (at 139.8 96.024) (size 0.55) (drill 0.3) (layers "F.Cu" "B.Cu") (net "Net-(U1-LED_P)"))
 (segment (start 139.8 81) (end 145.412 81) (width 0.25) (layer "B.Cu") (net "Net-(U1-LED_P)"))
 (segment (start 139.8 96.024) (end 139.8 81) (width 0.25) (layer "B.Cu") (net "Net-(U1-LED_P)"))
 (segment (start 145.412 81) (end 145.412 82.5) (width 0.25) (layer "B.Cu") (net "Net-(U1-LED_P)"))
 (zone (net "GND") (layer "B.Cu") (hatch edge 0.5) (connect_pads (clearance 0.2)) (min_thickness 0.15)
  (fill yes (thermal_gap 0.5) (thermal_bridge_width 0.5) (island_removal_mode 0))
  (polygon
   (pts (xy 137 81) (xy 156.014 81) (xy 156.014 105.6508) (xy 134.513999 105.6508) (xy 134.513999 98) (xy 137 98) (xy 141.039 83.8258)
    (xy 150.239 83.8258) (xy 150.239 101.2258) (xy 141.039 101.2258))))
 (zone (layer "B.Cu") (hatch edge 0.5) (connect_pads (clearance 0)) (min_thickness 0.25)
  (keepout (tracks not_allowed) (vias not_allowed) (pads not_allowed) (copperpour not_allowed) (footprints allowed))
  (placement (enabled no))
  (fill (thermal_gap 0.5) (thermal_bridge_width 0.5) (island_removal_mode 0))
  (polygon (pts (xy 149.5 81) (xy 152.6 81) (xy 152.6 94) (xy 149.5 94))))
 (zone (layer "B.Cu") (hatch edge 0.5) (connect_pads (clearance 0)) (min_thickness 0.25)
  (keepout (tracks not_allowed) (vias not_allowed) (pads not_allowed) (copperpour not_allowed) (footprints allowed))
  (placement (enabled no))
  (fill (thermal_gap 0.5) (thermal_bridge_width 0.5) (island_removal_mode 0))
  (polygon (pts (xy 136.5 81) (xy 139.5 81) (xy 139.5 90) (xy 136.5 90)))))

